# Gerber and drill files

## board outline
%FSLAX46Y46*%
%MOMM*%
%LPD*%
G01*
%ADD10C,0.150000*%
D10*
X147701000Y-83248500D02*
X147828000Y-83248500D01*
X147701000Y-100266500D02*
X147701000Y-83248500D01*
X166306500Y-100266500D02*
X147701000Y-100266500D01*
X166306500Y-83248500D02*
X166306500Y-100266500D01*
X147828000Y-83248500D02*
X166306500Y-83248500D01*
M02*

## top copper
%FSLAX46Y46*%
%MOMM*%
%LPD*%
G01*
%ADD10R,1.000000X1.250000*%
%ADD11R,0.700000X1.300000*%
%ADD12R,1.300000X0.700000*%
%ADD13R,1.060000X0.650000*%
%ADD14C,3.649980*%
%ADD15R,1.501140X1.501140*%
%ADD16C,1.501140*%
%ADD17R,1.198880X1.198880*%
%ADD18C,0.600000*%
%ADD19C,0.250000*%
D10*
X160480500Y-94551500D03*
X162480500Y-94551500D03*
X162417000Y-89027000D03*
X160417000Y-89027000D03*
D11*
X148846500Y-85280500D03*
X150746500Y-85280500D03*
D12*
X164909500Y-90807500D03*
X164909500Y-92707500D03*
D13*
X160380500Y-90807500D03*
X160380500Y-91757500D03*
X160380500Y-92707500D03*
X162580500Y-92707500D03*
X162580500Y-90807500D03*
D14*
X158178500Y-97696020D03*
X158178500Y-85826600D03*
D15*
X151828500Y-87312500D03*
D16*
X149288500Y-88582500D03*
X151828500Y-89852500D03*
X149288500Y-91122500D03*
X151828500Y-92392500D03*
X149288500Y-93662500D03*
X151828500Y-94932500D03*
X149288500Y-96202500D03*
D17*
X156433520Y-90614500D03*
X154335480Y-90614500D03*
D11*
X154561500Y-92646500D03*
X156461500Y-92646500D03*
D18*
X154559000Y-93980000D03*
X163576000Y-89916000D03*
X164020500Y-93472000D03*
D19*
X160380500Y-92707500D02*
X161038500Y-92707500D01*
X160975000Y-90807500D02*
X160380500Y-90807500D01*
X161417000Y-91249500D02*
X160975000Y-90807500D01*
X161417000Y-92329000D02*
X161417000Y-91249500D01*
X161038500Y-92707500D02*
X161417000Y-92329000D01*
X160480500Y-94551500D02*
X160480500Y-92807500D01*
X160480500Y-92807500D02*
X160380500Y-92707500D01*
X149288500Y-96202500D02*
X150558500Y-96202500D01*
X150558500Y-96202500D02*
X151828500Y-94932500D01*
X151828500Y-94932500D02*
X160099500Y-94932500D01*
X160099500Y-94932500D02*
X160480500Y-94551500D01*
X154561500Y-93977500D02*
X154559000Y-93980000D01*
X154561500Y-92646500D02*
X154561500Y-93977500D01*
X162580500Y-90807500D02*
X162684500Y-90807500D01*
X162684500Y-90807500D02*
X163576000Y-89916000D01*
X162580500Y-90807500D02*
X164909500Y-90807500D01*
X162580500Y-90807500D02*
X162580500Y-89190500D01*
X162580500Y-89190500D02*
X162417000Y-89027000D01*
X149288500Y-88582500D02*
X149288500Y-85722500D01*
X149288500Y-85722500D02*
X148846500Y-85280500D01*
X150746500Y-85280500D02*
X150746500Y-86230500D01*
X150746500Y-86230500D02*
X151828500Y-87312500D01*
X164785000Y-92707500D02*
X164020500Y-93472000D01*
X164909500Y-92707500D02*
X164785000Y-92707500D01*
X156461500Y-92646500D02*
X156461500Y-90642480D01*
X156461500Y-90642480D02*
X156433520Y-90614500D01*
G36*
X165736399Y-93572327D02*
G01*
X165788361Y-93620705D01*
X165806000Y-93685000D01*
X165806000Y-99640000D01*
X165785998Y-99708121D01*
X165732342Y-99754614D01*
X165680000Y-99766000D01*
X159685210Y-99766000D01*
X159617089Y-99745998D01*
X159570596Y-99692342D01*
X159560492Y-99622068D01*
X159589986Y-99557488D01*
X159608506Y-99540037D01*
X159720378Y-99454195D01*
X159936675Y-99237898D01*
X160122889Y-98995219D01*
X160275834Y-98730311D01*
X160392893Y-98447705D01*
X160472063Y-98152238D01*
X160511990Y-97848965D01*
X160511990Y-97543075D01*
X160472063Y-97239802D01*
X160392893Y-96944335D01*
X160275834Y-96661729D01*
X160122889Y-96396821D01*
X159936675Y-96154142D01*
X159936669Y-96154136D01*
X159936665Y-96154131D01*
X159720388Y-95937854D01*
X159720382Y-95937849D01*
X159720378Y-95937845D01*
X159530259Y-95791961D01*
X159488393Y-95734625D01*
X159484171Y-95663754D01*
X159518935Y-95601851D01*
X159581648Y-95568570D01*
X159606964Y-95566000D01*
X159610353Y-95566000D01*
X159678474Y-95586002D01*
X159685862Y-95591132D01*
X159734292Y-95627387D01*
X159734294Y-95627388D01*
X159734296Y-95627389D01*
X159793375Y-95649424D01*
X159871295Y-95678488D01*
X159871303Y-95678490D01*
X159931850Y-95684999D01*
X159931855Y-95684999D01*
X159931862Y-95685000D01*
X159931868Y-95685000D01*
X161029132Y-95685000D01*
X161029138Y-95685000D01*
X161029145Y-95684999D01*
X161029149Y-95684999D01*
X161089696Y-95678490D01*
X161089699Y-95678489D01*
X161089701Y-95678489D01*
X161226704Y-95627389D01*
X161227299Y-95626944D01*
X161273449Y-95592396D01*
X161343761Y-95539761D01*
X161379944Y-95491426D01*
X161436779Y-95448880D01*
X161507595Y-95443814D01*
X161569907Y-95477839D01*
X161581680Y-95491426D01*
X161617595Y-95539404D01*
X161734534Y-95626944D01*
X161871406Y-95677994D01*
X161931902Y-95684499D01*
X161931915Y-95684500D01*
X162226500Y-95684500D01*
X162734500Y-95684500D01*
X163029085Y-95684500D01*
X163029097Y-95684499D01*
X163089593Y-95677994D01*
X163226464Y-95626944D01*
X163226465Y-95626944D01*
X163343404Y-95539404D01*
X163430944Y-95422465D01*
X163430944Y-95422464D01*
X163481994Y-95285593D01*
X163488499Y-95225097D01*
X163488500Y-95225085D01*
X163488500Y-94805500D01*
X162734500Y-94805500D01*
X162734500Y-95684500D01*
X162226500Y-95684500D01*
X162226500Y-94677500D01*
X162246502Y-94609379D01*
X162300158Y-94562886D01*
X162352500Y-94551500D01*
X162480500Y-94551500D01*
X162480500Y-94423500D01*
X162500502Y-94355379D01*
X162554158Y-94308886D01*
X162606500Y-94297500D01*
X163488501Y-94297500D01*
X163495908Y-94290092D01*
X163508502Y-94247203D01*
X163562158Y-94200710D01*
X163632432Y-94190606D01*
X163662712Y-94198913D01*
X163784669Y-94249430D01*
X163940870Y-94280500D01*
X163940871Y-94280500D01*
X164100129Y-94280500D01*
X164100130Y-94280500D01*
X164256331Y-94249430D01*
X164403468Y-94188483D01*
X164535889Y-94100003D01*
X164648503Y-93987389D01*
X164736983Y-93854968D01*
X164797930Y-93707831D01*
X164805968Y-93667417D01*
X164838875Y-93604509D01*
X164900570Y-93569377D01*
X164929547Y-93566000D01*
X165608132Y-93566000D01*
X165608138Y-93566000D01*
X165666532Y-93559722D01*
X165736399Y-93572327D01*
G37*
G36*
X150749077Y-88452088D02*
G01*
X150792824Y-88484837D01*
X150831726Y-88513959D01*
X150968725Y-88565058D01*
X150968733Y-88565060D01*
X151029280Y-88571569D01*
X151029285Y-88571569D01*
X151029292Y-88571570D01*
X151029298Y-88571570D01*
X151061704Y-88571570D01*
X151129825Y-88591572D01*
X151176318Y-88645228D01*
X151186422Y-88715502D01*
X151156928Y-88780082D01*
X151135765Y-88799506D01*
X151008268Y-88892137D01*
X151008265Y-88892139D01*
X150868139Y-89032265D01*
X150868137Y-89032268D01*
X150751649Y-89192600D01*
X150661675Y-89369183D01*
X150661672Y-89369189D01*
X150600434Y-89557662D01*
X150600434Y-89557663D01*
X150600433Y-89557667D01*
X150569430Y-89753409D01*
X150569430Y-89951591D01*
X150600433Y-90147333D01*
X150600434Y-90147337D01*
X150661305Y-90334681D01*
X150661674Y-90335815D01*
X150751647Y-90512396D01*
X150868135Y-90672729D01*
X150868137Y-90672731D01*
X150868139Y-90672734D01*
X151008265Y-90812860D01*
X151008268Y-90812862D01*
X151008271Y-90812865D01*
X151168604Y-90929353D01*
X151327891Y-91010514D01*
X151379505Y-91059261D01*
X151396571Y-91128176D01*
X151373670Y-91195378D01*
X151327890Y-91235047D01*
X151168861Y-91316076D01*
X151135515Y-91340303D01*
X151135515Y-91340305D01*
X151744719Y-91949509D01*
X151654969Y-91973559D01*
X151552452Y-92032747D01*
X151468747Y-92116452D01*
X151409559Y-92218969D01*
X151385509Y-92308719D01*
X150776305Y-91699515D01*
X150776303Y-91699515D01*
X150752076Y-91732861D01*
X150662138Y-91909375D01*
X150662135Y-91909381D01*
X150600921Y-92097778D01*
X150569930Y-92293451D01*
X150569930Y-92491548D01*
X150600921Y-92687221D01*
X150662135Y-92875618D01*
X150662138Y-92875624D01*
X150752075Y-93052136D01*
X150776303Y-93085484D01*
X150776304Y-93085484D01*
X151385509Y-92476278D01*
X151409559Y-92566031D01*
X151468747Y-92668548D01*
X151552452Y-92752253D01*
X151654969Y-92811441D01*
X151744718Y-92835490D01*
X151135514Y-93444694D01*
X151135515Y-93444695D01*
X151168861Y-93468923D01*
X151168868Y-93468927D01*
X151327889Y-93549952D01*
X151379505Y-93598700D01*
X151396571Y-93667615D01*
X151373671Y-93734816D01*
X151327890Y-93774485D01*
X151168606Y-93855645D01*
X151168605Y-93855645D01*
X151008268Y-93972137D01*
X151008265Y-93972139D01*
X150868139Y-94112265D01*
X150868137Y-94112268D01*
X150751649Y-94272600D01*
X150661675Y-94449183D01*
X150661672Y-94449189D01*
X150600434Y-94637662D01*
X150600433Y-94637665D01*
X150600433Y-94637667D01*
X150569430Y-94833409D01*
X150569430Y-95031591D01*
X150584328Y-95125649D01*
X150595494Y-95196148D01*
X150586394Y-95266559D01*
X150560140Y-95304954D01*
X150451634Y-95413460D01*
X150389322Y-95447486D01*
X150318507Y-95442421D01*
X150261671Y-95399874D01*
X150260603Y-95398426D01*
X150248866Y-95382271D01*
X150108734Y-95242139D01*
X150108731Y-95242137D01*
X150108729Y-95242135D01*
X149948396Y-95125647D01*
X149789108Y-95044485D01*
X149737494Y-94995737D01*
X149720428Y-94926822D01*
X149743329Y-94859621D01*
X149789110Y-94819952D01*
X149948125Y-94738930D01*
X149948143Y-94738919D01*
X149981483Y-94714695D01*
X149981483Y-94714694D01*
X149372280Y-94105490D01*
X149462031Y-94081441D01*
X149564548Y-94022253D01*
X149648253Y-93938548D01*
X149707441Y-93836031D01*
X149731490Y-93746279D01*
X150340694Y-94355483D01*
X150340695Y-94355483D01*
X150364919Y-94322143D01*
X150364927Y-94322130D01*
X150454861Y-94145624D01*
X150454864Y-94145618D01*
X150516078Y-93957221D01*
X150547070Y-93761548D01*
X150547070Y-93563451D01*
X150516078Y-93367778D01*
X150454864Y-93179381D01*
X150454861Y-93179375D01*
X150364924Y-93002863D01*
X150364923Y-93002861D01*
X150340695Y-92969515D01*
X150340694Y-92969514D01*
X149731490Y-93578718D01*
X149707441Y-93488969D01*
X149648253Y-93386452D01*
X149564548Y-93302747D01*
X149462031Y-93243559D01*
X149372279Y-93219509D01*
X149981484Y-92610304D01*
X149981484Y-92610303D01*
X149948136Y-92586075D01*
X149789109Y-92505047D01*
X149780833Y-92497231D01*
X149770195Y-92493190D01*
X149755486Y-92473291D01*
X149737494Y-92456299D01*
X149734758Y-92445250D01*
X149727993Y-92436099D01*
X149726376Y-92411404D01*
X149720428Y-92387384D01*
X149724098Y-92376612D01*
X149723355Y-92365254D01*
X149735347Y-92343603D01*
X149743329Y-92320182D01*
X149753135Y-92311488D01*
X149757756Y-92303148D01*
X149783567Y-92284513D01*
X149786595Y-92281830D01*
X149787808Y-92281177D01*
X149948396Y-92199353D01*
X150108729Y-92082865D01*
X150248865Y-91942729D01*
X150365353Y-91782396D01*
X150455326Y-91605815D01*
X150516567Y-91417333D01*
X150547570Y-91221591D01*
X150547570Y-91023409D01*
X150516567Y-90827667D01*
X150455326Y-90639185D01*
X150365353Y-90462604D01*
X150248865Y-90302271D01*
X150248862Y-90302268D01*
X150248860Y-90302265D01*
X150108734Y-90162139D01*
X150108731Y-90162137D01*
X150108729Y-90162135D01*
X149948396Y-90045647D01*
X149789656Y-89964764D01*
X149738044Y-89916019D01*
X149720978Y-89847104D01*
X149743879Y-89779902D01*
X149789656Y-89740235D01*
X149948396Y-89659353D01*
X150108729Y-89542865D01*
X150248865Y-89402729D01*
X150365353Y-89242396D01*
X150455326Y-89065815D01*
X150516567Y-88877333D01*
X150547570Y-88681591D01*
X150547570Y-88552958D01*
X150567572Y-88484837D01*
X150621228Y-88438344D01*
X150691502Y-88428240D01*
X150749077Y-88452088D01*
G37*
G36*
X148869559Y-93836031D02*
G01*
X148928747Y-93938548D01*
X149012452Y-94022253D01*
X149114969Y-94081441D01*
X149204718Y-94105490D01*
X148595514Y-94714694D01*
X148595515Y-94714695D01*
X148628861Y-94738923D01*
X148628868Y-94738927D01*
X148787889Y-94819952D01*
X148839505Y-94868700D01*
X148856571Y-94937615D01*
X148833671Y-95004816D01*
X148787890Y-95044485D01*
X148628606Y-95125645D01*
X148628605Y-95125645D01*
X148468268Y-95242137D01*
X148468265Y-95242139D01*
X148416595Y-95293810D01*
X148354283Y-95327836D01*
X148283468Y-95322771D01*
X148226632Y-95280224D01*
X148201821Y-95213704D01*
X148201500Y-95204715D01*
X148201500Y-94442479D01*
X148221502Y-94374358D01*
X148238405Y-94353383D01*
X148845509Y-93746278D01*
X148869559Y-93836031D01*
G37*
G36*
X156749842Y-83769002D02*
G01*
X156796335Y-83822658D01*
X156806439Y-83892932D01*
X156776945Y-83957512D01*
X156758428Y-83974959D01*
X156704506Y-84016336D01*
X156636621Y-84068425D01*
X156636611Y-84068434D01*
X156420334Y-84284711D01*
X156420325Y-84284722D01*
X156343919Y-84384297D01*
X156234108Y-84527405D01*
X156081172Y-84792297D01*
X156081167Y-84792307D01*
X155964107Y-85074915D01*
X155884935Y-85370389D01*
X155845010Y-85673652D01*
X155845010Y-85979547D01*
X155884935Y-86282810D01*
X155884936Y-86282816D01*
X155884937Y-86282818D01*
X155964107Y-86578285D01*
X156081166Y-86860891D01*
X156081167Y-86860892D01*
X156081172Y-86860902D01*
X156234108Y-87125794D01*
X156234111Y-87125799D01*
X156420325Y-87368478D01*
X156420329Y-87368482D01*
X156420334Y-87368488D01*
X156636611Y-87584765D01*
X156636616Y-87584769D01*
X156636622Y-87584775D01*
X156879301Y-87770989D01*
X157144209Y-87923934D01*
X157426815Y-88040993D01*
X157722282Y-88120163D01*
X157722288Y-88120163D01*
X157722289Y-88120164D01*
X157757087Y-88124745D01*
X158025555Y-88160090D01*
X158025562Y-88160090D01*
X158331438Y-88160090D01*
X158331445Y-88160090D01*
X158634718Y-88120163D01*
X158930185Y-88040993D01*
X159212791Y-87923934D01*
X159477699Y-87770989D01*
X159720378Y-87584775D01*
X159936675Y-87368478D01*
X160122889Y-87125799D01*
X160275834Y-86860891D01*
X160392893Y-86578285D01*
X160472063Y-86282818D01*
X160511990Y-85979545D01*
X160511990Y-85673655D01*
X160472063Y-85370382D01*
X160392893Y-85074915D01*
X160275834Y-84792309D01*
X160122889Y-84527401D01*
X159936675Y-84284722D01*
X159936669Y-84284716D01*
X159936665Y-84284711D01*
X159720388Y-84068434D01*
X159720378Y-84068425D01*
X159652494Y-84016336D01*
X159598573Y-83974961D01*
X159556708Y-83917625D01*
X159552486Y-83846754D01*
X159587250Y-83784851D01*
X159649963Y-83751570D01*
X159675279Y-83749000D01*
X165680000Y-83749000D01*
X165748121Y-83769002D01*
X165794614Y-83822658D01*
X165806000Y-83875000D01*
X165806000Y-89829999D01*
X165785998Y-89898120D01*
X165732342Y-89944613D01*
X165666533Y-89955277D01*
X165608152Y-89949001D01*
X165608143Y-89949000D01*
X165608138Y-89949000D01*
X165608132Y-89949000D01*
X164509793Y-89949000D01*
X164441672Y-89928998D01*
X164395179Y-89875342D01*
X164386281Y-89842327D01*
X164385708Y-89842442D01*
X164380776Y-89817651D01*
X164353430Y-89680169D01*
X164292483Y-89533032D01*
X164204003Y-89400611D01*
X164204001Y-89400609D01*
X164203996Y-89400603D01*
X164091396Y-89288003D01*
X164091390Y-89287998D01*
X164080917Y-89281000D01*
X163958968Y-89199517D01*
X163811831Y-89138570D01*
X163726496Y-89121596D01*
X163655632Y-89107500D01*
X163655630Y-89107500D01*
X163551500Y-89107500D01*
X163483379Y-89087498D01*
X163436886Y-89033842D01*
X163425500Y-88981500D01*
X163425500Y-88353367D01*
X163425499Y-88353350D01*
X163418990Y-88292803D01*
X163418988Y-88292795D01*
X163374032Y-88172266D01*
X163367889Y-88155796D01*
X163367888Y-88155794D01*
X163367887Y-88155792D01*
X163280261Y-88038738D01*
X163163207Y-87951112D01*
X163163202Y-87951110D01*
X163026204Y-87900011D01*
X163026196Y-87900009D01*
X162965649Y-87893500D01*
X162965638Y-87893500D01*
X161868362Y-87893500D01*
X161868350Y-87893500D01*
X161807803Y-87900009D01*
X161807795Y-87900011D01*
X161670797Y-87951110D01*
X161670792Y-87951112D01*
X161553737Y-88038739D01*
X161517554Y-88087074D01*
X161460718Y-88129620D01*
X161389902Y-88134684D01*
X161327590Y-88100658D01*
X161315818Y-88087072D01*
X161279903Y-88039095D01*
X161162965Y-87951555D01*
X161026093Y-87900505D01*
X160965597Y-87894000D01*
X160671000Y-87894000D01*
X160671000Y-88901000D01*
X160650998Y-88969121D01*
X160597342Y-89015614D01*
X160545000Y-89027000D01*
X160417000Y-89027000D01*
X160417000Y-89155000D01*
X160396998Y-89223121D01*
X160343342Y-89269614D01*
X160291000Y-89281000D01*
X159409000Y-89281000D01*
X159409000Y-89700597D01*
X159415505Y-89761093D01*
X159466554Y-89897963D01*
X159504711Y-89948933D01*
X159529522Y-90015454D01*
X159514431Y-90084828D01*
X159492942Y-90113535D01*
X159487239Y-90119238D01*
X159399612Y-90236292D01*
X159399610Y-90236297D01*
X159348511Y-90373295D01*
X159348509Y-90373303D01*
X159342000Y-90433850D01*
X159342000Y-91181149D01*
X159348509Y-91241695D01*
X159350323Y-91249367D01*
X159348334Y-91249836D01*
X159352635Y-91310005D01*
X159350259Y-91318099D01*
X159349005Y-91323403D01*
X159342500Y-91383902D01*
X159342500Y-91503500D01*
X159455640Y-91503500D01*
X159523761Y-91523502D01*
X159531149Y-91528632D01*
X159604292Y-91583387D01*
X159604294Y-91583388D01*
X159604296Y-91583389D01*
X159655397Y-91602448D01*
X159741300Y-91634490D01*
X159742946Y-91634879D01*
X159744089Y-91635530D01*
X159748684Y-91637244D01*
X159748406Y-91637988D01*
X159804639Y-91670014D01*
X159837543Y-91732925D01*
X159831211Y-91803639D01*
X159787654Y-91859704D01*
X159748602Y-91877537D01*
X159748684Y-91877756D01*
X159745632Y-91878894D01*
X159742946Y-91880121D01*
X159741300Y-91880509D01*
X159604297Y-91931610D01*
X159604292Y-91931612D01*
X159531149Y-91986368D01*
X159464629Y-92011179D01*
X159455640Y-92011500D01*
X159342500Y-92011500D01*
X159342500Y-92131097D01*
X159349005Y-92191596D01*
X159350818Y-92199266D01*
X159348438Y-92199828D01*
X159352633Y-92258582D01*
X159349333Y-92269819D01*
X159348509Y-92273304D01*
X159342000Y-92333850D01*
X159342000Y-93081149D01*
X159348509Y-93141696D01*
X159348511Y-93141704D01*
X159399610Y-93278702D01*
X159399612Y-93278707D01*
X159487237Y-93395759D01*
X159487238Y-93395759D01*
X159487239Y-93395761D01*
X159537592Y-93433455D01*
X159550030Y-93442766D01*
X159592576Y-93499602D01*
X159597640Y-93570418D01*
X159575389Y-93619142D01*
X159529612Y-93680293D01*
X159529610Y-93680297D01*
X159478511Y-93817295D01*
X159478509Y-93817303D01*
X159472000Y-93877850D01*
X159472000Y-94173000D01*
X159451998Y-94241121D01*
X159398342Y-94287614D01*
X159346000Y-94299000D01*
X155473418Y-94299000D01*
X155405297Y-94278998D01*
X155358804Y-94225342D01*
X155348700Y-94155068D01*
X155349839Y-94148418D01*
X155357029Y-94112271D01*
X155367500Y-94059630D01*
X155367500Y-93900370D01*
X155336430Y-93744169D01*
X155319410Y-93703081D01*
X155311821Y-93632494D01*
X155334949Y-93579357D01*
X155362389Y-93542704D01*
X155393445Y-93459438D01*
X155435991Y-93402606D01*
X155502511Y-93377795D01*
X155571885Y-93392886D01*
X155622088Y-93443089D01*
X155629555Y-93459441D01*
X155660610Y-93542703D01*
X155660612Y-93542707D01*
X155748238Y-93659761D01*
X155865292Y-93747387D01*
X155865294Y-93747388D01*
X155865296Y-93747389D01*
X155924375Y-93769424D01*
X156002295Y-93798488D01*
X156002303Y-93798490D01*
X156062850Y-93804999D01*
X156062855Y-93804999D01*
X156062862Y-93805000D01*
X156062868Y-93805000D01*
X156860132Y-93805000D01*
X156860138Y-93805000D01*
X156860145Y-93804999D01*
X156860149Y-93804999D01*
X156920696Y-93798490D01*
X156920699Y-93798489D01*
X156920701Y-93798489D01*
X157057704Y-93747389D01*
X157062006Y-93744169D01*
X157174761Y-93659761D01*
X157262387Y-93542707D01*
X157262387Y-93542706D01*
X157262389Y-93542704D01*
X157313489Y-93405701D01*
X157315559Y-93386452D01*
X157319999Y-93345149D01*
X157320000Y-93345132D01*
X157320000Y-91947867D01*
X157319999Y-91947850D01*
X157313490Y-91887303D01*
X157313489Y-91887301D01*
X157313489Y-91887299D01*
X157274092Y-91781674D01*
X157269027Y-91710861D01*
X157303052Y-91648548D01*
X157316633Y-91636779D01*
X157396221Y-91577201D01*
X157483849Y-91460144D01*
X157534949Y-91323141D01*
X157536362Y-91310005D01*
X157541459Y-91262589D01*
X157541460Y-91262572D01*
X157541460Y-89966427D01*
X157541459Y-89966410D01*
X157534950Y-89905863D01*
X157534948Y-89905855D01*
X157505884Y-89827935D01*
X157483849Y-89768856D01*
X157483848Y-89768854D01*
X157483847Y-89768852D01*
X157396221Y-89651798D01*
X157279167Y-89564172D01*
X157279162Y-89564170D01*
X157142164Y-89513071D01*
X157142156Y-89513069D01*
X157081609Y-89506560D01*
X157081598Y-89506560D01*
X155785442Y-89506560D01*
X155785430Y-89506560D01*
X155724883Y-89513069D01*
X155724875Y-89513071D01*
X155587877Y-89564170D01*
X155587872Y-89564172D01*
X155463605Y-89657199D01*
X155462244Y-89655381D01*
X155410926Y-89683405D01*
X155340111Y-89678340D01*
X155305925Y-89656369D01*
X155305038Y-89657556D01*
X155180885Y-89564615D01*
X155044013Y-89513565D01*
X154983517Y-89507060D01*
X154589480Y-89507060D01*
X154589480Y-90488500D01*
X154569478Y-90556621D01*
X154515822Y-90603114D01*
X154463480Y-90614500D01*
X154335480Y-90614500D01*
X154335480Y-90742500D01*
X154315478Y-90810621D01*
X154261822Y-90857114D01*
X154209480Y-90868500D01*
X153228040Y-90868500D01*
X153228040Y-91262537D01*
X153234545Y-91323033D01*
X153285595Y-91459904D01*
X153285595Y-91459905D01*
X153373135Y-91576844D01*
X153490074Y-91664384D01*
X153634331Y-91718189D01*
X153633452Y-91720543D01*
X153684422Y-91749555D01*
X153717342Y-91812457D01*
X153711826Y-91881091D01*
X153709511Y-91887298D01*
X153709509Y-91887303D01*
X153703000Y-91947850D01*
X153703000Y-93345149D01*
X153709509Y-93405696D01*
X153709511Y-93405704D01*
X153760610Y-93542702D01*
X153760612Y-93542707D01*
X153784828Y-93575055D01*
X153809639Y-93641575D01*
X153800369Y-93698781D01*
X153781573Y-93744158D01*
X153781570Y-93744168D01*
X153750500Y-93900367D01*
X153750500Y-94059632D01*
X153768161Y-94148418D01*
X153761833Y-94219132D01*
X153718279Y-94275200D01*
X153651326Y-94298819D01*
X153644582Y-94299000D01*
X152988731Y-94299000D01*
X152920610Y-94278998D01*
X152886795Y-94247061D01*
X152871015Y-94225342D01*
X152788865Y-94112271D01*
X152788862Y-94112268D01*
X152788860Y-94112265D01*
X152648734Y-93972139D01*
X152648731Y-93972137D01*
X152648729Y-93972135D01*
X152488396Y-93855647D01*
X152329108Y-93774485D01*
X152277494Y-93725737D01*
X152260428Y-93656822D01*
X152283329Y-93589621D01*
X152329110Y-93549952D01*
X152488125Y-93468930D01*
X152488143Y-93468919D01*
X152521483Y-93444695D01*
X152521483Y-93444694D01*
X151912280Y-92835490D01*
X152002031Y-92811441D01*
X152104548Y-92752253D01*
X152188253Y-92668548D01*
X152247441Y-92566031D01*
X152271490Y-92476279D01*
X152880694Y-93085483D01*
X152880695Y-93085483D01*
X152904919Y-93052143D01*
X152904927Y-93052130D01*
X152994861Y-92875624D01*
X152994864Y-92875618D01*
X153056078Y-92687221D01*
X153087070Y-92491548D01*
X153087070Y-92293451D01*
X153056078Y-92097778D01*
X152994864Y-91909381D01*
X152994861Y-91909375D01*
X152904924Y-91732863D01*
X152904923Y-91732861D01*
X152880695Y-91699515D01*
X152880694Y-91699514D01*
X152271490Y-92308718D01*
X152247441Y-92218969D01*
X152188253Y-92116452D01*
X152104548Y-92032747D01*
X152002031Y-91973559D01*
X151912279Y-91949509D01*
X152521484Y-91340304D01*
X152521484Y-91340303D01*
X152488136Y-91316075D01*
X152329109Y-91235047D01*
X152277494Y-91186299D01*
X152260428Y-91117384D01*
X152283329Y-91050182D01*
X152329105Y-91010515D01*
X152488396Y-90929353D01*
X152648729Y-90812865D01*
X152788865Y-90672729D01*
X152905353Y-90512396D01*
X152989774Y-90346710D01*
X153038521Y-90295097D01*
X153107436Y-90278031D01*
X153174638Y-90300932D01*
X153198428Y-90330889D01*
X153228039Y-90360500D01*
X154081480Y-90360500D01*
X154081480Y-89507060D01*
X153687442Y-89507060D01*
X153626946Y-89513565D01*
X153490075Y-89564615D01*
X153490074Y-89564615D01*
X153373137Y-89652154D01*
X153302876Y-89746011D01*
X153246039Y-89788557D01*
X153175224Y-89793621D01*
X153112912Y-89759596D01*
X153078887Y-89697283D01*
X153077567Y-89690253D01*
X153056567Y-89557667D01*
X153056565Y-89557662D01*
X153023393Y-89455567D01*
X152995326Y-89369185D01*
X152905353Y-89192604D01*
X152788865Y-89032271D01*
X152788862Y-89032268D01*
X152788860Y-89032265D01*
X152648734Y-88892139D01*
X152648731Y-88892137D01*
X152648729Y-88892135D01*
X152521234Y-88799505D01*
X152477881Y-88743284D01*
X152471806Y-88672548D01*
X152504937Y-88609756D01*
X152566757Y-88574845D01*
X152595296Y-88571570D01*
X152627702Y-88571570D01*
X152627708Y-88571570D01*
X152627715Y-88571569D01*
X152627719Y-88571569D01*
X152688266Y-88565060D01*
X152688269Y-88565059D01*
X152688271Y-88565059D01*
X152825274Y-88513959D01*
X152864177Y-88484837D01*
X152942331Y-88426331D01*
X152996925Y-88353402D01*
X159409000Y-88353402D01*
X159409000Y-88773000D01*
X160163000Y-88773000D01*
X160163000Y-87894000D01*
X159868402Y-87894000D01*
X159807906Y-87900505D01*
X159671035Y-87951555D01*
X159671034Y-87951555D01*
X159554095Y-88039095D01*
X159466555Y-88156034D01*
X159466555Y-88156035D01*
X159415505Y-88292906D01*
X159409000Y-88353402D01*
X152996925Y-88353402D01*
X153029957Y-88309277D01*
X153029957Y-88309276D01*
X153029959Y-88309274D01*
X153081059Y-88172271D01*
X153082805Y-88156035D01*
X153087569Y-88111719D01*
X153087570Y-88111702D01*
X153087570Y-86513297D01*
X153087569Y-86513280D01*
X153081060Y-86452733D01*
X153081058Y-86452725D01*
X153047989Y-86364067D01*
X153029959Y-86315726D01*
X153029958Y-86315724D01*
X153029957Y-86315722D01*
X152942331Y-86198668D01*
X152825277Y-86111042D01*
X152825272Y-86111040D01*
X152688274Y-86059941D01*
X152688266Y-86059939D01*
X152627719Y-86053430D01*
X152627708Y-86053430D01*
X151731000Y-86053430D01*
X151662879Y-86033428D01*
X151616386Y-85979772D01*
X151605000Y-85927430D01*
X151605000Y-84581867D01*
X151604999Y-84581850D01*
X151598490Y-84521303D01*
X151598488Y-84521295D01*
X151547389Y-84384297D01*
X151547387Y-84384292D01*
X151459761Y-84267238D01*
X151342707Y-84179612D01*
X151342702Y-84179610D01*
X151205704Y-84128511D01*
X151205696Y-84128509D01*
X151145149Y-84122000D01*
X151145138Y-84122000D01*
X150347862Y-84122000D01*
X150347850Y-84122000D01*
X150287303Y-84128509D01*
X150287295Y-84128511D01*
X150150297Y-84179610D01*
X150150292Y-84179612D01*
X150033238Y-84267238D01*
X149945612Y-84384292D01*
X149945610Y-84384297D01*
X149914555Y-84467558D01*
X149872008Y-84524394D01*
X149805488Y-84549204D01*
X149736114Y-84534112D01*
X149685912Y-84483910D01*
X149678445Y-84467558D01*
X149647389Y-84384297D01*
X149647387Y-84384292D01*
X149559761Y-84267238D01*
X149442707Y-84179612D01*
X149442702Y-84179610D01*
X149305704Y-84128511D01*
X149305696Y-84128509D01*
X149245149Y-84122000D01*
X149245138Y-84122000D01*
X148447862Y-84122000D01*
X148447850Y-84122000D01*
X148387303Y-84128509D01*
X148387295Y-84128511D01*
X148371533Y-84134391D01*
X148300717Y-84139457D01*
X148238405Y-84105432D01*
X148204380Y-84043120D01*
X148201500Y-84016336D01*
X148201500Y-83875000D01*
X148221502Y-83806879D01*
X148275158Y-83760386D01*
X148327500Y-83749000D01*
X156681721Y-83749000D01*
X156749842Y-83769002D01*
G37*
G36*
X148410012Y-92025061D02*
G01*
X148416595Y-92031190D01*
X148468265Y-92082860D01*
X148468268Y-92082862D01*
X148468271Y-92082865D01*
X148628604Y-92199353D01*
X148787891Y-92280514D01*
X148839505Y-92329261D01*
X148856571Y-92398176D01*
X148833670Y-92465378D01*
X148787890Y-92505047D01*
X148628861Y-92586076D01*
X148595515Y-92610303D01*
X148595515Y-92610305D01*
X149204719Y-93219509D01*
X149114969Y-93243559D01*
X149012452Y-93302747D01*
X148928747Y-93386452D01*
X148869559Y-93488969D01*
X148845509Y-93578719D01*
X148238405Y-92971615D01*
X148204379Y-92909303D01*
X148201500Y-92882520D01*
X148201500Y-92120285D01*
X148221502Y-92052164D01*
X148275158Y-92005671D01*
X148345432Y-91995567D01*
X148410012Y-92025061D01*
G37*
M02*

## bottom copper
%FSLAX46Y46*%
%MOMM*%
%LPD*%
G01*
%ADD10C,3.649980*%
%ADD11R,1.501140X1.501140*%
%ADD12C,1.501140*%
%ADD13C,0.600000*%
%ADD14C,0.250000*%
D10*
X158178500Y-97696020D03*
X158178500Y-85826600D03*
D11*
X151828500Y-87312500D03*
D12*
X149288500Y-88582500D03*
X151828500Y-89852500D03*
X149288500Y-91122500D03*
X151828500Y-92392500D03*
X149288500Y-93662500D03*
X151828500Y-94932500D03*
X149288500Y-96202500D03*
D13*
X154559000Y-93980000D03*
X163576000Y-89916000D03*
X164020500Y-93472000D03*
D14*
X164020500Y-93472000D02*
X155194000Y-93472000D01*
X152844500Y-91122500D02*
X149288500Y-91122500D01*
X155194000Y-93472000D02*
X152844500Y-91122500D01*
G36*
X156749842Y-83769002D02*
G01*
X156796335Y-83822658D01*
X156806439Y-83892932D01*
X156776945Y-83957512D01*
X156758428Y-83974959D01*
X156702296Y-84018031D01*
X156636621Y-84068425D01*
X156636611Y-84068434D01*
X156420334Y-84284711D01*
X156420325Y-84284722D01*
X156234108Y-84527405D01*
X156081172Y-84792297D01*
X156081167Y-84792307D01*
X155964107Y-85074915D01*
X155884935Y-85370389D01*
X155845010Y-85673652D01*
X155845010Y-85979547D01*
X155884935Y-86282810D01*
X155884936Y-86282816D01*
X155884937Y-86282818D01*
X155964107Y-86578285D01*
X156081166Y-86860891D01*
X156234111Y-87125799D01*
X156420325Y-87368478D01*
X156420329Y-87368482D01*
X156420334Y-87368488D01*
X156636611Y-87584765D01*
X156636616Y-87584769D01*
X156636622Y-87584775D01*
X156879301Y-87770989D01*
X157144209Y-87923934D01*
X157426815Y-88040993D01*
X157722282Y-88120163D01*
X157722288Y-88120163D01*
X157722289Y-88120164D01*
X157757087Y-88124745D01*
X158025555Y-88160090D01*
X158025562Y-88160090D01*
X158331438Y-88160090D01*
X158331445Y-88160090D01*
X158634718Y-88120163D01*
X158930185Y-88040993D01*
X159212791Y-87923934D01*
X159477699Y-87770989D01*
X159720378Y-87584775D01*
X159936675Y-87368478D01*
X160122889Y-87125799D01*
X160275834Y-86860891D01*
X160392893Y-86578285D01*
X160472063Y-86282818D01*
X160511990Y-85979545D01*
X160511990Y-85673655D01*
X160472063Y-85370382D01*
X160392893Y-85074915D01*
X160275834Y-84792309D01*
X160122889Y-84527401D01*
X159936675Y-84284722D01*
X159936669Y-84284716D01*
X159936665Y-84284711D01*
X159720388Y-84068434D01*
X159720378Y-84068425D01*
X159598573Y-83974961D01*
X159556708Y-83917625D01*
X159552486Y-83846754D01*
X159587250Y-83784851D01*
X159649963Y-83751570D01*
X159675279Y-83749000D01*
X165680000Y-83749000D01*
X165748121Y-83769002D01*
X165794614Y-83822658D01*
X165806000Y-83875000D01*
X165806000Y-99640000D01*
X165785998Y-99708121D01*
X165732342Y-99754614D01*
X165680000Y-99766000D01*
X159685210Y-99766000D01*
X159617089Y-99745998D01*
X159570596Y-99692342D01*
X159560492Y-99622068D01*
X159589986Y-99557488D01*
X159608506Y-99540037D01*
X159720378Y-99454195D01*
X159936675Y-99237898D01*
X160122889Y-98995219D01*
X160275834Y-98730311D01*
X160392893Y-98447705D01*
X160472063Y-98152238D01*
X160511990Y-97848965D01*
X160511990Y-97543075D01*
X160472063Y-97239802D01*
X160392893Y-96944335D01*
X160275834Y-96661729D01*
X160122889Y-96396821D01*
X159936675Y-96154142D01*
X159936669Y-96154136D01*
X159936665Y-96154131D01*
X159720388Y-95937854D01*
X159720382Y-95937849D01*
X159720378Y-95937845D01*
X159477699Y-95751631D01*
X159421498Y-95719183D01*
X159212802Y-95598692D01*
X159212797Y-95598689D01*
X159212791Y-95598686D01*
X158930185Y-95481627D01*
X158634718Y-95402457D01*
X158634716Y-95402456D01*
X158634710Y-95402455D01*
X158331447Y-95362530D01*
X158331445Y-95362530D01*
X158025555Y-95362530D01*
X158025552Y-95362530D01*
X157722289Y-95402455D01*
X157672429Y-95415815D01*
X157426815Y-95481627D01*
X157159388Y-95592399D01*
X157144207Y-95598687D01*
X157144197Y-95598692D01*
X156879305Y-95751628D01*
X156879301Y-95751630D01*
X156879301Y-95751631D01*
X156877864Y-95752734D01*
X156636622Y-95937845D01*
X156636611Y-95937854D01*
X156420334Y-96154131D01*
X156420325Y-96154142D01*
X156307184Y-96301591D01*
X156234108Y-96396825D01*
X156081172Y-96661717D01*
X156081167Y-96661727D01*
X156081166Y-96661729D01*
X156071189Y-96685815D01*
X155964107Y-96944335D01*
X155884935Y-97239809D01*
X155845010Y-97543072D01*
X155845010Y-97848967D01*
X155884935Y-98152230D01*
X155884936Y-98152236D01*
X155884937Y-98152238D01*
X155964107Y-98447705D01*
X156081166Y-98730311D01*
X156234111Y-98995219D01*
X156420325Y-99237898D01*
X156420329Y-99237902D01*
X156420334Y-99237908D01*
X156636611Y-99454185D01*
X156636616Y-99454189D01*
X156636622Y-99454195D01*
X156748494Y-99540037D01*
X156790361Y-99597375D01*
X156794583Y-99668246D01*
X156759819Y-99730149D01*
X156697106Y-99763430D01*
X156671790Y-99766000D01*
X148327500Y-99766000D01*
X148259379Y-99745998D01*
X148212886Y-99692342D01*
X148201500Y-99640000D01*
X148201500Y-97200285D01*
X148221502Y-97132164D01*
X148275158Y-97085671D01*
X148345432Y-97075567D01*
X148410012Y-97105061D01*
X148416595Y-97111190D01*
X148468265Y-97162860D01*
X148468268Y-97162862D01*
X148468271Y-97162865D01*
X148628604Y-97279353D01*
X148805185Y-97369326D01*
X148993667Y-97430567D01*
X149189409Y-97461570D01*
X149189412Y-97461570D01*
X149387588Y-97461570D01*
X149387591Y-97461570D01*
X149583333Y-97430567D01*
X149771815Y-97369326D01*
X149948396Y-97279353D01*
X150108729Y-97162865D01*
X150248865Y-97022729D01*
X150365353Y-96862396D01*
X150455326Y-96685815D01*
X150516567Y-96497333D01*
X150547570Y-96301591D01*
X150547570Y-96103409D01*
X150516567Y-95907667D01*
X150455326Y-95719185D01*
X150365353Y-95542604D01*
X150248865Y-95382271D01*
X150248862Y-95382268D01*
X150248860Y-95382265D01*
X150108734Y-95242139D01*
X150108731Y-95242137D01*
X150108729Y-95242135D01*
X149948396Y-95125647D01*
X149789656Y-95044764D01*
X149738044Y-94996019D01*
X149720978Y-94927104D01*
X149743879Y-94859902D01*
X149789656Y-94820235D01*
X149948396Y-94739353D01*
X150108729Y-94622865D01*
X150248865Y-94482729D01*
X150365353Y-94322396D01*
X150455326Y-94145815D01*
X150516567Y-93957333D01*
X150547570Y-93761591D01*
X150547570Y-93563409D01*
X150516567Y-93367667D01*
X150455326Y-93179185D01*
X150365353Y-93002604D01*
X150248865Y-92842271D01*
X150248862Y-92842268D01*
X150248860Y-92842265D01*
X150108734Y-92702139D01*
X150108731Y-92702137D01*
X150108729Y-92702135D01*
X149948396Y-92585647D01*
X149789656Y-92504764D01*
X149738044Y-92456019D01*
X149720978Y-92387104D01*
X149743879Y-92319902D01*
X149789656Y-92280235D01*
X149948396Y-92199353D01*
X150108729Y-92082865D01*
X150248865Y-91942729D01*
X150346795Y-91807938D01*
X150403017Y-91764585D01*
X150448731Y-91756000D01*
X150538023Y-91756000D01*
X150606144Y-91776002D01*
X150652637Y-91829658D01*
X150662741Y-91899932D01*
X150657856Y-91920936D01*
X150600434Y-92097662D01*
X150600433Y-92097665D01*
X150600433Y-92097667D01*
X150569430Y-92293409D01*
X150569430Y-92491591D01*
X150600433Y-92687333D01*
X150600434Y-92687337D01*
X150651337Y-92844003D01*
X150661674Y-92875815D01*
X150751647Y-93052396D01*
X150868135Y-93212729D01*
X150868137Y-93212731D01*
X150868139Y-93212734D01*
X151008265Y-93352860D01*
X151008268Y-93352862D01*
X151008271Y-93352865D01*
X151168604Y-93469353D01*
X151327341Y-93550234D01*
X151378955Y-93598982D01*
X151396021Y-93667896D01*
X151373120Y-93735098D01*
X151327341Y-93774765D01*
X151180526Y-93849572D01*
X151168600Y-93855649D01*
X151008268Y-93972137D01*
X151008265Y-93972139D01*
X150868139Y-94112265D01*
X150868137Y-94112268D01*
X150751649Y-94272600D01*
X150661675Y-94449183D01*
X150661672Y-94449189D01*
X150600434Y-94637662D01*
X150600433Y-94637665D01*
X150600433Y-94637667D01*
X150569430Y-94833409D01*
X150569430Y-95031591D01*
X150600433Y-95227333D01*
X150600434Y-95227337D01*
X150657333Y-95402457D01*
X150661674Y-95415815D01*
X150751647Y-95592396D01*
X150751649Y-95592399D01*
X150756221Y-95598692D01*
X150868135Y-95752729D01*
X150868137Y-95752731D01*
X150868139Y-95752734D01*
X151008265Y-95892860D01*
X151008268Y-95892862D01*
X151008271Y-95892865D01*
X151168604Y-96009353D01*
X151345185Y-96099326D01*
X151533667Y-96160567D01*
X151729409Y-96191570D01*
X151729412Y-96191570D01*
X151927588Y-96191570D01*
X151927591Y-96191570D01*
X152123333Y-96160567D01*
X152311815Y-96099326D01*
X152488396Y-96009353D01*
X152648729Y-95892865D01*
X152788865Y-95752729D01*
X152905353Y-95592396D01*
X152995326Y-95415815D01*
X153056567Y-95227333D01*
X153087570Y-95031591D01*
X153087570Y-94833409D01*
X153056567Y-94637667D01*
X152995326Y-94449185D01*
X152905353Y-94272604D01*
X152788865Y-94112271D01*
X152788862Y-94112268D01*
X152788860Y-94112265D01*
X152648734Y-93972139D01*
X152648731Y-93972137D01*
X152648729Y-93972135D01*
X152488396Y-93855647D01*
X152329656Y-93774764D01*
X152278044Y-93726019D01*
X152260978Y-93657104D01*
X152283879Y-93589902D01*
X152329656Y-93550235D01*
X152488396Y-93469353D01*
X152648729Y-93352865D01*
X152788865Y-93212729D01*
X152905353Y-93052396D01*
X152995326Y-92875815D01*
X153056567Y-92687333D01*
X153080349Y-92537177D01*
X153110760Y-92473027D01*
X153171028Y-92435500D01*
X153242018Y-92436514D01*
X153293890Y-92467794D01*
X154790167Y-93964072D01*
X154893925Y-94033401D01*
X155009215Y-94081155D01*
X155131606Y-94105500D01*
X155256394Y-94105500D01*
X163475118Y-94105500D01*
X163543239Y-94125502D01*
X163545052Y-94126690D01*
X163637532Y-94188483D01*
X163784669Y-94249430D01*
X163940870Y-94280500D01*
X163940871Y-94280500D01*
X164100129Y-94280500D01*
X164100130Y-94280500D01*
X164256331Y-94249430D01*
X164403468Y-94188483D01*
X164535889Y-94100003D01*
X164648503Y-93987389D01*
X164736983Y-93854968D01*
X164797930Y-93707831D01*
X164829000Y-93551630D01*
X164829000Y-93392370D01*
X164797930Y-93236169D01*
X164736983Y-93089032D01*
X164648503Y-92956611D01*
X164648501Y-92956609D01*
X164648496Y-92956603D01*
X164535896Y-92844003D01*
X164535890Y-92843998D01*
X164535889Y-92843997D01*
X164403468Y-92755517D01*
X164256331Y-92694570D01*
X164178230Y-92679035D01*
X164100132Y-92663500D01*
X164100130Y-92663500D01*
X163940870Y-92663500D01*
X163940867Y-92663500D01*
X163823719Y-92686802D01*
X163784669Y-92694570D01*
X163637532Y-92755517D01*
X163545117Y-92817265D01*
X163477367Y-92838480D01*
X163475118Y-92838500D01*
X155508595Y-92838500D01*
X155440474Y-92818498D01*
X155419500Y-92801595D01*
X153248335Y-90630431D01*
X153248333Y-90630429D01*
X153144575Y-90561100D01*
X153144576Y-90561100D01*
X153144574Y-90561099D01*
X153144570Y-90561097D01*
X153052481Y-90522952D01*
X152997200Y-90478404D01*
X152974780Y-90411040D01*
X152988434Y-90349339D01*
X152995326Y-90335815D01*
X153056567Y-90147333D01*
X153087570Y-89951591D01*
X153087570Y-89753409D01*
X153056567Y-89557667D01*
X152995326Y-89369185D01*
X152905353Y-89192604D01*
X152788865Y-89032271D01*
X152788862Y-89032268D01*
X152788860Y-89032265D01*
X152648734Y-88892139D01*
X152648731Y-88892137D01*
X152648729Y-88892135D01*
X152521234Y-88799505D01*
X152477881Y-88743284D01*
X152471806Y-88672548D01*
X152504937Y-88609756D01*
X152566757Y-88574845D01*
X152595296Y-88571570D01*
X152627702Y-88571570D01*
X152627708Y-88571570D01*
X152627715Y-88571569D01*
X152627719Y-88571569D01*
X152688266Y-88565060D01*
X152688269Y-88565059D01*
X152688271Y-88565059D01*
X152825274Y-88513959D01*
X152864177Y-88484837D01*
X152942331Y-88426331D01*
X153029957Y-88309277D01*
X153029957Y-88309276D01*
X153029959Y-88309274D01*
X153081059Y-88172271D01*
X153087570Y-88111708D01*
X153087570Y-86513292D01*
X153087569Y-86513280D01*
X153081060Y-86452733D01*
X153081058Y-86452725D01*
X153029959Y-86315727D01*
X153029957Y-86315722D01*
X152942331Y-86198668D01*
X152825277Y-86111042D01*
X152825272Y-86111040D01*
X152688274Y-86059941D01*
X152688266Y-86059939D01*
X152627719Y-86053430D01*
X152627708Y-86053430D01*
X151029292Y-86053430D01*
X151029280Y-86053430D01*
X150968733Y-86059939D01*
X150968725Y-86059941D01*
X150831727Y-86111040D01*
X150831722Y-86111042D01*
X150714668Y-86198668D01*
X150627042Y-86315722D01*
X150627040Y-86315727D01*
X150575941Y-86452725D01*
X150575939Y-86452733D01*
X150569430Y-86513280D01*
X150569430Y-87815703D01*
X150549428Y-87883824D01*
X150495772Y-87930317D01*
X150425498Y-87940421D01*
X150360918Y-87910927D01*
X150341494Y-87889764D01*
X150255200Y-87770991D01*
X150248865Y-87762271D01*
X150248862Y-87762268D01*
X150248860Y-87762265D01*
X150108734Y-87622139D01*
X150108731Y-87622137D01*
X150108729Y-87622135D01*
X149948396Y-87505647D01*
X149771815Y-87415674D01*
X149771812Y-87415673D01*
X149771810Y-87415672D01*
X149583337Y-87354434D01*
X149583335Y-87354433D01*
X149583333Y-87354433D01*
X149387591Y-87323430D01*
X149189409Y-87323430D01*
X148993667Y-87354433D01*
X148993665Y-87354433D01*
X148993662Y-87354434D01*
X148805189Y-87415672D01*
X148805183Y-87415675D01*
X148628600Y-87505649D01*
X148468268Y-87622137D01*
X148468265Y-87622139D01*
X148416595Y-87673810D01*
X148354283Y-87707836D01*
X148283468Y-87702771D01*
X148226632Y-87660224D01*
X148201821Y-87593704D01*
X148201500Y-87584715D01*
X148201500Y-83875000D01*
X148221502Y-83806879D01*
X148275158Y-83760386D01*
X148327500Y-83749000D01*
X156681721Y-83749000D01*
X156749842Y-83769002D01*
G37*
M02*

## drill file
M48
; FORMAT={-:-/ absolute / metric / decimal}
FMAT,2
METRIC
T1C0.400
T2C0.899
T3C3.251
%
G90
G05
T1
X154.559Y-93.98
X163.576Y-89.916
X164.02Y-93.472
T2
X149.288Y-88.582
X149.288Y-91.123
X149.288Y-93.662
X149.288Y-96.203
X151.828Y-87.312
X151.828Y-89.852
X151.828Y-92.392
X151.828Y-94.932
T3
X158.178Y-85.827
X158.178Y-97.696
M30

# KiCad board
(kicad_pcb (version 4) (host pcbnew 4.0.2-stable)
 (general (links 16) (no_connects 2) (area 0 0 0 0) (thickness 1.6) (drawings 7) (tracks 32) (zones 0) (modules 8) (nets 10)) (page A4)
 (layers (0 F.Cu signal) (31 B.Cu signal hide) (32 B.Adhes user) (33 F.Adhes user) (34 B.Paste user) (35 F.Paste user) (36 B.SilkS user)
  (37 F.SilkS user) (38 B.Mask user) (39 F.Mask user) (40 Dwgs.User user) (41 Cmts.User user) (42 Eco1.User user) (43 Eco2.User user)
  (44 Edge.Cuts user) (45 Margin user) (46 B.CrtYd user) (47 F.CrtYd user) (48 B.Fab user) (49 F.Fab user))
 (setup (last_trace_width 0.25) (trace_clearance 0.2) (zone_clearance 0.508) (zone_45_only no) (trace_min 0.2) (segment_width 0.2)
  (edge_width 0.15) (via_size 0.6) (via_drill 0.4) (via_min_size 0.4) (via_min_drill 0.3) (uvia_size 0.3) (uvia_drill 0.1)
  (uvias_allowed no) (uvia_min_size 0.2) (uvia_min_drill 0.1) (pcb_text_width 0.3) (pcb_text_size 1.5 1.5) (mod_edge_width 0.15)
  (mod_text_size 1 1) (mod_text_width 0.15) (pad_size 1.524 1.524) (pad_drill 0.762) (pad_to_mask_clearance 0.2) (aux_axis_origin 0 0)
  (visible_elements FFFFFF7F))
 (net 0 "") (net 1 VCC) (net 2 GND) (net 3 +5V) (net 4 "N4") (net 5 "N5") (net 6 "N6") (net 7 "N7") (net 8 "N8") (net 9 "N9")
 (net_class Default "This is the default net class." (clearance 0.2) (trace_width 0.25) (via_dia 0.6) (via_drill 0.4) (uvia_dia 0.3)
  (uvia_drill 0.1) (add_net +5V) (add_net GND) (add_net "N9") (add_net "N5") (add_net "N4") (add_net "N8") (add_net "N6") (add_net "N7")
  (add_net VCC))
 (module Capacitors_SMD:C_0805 (layer F.Cu) (at 161.4805 94.5515)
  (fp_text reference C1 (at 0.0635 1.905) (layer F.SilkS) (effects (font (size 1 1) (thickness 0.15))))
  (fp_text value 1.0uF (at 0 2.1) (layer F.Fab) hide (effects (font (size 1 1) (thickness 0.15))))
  (pad 1 smd rect (at -1 0) (size 1 1.25) (layers F.Cu F.Paste F.Mask) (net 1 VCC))
  (pad 2 smd rect (at 1 0) (size 1 1.25) (layers F.Cu F.Paste F.Mask) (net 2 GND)))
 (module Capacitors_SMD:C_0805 (layer F.Cu) (at 161.417 89.027 180)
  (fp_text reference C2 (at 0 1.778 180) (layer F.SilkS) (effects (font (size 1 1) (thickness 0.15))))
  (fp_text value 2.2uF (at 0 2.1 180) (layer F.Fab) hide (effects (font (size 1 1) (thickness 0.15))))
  (pad 1 smd rect (at -1 0 180) (size 1 1.25) (layers F.Cu F.Paste F.Mask) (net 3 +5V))
  (pad 2 smd rect (at 1 0 180) (size 1 1.25) (layers F.Cu F.Paste F.Mask) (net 2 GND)))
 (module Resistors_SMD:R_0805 (layer F.Cu) (at 149.7965 85.2805)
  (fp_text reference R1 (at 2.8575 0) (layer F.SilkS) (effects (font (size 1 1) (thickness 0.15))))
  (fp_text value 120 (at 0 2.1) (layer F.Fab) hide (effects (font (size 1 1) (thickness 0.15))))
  (pad 1 smd rect (at -0.95 0) (size 0.7 1.3) (layers F.Cu F.Paste F.Mask) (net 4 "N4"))
  (pad 2 smd rect (at 0.95 0) (size 0.7 1.3) (layers F.Cu F.Paste F.Mask) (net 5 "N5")))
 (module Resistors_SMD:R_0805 (layer F.Cu) (at 164.9095 91.7575 270)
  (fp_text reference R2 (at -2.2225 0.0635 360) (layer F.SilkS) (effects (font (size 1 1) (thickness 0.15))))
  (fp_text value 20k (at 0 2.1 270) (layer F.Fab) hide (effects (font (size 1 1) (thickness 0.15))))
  (pad 1 smd rect (at -0.95 0 270) (size 0.7 1.3) (layers F.Cu F.Paste F.Mask) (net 3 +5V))
  (pad 2 smd rect (at 0.95 0 270) (size 0.7 1.3) (layers F.Cu F.Paste F.Mask) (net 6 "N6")))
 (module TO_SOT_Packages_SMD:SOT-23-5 (layer F.Cu) (at 161.4805 91.7575)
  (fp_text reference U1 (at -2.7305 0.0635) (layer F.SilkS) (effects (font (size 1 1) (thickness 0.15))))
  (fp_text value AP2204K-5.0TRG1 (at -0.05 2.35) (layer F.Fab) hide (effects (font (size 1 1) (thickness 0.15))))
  (pad 1 smd rect (at -1.1 -0.95) (size 1.06 0.65) (layers F.Cu F.Paste F.Mask) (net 1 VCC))
  (pad 2 smd rect (at -1.1 0) (size 1.06 0.65) (layers F.Cu F.Paste F.Mask) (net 2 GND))
  (pad 3 smd rect (at -1.1 0.95) (size 1.06 0.65) (layers F.Cu F.Paste F.Mask) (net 1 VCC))
  (pad 4 smd rect (at 1.1 0.95) (size 1.06 0.65) (layers F.Cu F.Paste F.Mask) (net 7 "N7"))
  (pad 5 smd rect (at 1.1 -0.95) (size 1.06 0.65) (layers F.Cu F.Paste F.Mask) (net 3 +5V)))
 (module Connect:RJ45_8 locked (layer B.Cu) (at 158.1785 91.7575 270)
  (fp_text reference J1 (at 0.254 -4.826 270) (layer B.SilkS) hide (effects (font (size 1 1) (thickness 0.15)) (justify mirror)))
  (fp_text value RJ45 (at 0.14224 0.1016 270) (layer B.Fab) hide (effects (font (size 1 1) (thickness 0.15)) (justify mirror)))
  (pad Hole np_thru_hole circle (at 5.93852 0 270) (size 3.64998 3.64998) (drill 3.2512) (layers *.Cu *.SilkS *.Mask))
  (pad Hole np_thru_hole circle (at -5.9309 0 270) (size 3.64998 3.64998) (drill 3.2512) (layers *.Cu *.SilkS *.Mask))
  (pad 1 thru_hole rect (at -4.445 6.35 270) (size 1.50114 1.50114) (drill 0.89916) (layers *.Cu *.Mask B.SilkS) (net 5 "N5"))
  (pad 2 thru_hole circle (at -3.175 8.89 270) (size 1.50114 1.50114) (drill 0.89916) (layers *.Cu *.Mask B.SilkS) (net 4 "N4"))
  (pad 3 thru_hole circle (at -1.905 6.35 270) (size 1.50114 1.50114) (drill 0.89916) (layers *.Cu *.Mask B.SilkS) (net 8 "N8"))
  (pad 4 thru_hole circle (at -0.635 8.89 270) (size 1.50114 1.50114) (drill 0.89916) (layers *.Cu *.Mask B.SilkS) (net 6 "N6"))
  (pad 5 thru_hole circle (at 0.635 6.35 270) (size 1.50114 1.50114) (drill 0.89916) (layers *.Cu *.Mask B.SilkS) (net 2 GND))
  (pad 6 thru_hole circle (at 1.905 8.89 270) (size 1.50114 1.50114) (drill 0.89916) (layers *.Cu *.Mask B.SilkS) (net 2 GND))
  (pad 7 thru_hole circle (at 3.175 6.35 270) (size 1.50114 1.50114) (drill 0.89916) (layers *.Cu *.Mask B.SilkS) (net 1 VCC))
  (pad 8 thru_hole circle (at 4.445 8.89 270) (size 1.50114 1.50114) (drill 0.89916) (layers *.Cu *.Mask B.SilkS) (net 1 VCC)))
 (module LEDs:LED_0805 (layer F.Cu) (at 155.3845 90.6145)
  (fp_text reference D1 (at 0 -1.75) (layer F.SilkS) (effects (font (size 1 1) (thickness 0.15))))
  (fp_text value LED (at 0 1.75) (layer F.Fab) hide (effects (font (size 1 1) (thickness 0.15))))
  (pad 2 smd rect (at 1.04902 0 180) (size 1.19888 1.19888) (layers F.Cu F.Paste F.Mask) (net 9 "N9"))
  (pad 1 smd rect (at -1.04902 0 180) (size 1.19888 1.19888) (layers F.Cu F.Paste F.Mask) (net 2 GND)))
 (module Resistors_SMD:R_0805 (layer F.Cu) (at 155.5115 92.6465)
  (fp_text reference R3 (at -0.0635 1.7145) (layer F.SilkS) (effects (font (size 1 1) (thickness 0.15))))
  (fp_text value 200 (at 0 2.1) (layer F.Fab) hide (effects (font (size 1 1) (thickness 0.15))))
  (pad 1 smd rect (at -0.95 0) (size 0.7 1.3) (layers F.Cu F.Paste F.Mask) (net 3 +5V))
  (pad 2 smd rect (at 0.95 0) (size 0.7 1.3) (layers F.Cu F.Paste F.Mask) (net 9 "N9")))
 (gr_line (start 147.701 83.2485) (end 147.828 83.2485) (angle 90) (layer Edge.Cuts) (width 0.15))
 (gr_line (start 147.701 100.2665) (end 147.701 83.2485) (angle 90) (layer Edge.Cuts) (width 0.15))
 (gr_line (start 166.3065 100.2665) (end 147.701 100.2665) (angle 90) (layer Edge.Cuts) (width 0.15))
 (gr_line (start 166.3065 83.2485) (end 166.3065 100.2665) (angle 90) (layer Edge.Cuts) (width 0.15))
 (gr_line (start 147.828 83.2485) (end 166.3065 83.2485) (angle 90) (layer Edge.Cuts) (width 0.15))
 (segment (start 160.3805 92.7075) (end 161.0385 92.7075) (width 0.25) (layer F.Cu) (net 1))
 (segment (start 160.975 90.8075) (end 160.3805 90.8075) (width 0.25) (layer F.Cu) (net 1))
 (segment (start 161.417 91.2495) (end 160.975 90.8075) (width 0.25) (layer F.Cu) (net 1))
 (segment (start 161.417 92.329) (end 161.417 91.2495) (width 0.25) (layer F.Cu) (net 1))
 (segment (start 161.0385 92.7075) (end 161.417 92.329) (width 0.25) (layer F.Cu) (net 1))
 (segment (start 160.4805 94.5515) (end 160.4805 92.8075) (width 0.25) (layer F.Cu) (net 1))
 (segment (start 160.4805 92.8075) (end 160.3805 92.7075) (width 0.25) (layer F.Cu) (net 1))
 (segment (start 149.2885 96.2025) (end 150.5585 96.2025) (width 0.25) (layer F.Cu) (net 1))
 (segment (start 150.5585 96.2025) (end 151.8285 94.9325) (width 0.25) (layer F.Cu) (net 1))
 (segment (start 151.8285 94.9325) (end 160.0995 94.9325) (width 0.25) (layer F.Cu) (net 1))
 (segment (start 160.0995 94.9325) (end 160.4805 94.5515) (width 0.25) (layer F.Cu) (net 1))
 (via (at 154.559 93.98) (size 0.6) (drill 0.4) (layers F.Cu B.Cu) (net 3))
 (segment (start 154.5615 93.9775) (end 154.559 93.98) (width 0.25) (layer F.Cu) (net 3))
 (segment (start 154.5615 92.6465) (end 154.5615 93.9775) (width 0.25) (layer F.Cu) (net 3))
 (segment (start 162.5805 90.8075) (end 162.6845 90.8075) (width 0.25) (layer F.Cu) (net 3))
 (segment (start 162.6845 90.8075) (end 163.576 89.916) (width 0.25) (layer F.Cu) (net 3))
 (via (at 163.576 89.916) (size 0.6) (drill 0.4) (layers F.Cu B.Cu) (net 3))
 (segment (start 162.5805 90.8075) (end 164.9095 90.8075) (width 0.25) (layer F.Cu) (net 3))
 (segment (start 162.5805 90.8075) (end 162.5805 89.1905) (width 0.25) (layer F.Cu) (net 3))
 (segment (start 162.5805 89.1905) (end 162.417 89.027) (width 0.25) (layer F.Cu) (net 3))
 (segment (start 149.2885 88.5825) (end 149.2885 85.7225) (width 0.25) (layer F.Cu) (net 4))
 (segment (start 149.2885 85.7225) (end 148.8465 85.2805) (width 0.25) (layer F.Cu) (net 4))
 (segment (start 150.7465 85.2805) (end 150.7465 86.2305) (width 0.25) (layer F.Cu) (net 5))
 (segment (start 150.7465 86.2305) (end 151.8285 87.3125) (width 0.25) (layer F.Cu) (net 5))
 (segment (start 164.0205 93.472) (end 155.194 93.472) (width 0.25) (layer B.Cu) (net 6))
 (via (at 164.0205 93.472) (size 0.6) (drill 0.4) (layers F.Cu B.Cu) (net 6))
 (segment (start 164.785 92.7075) (end 164.0205 93.472) (width 0.25) (layer F.Cu) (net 6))
 (segment (start 152.8445 91.1225) (end 149.2885 91.1225) (width 0.25) (layer B.Cu) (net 6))
 (segment (start 155.194 93.472) (end 152.8445 91.1225) (width 0.25) (layer B.Cu) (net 6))
 (segment (start 164.9095 92.7075) (end 164.785 92.7075) (width 0.25) (layer F.Cu) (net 6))
 (segment (start 156.4615 92.6465) (end 156.4615 90.64248) (width 0.25) (layer F.Cu) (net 9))
 (segment (start 156.4615 90.64248) (end 156.43352 90.6145) (width 0.25) (layer F.Cu) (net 9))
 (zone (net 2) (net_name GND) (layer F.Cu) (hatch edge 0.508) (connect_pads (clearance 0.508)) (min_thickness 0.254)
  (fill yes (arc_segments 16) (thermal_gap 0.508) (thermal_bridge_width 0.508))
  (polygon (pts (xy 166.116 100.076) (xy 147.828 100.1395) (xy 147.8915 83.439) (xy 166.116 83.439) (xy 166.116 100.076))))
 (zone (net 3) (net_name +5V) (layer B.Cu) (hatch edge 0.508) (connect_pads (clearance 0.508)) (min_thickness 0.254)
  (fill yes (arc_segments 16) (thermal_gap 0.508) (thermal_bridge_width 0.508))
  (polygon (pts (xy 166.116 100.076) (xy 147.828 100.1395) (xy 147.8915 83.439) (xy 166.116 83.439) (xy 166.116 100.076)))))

